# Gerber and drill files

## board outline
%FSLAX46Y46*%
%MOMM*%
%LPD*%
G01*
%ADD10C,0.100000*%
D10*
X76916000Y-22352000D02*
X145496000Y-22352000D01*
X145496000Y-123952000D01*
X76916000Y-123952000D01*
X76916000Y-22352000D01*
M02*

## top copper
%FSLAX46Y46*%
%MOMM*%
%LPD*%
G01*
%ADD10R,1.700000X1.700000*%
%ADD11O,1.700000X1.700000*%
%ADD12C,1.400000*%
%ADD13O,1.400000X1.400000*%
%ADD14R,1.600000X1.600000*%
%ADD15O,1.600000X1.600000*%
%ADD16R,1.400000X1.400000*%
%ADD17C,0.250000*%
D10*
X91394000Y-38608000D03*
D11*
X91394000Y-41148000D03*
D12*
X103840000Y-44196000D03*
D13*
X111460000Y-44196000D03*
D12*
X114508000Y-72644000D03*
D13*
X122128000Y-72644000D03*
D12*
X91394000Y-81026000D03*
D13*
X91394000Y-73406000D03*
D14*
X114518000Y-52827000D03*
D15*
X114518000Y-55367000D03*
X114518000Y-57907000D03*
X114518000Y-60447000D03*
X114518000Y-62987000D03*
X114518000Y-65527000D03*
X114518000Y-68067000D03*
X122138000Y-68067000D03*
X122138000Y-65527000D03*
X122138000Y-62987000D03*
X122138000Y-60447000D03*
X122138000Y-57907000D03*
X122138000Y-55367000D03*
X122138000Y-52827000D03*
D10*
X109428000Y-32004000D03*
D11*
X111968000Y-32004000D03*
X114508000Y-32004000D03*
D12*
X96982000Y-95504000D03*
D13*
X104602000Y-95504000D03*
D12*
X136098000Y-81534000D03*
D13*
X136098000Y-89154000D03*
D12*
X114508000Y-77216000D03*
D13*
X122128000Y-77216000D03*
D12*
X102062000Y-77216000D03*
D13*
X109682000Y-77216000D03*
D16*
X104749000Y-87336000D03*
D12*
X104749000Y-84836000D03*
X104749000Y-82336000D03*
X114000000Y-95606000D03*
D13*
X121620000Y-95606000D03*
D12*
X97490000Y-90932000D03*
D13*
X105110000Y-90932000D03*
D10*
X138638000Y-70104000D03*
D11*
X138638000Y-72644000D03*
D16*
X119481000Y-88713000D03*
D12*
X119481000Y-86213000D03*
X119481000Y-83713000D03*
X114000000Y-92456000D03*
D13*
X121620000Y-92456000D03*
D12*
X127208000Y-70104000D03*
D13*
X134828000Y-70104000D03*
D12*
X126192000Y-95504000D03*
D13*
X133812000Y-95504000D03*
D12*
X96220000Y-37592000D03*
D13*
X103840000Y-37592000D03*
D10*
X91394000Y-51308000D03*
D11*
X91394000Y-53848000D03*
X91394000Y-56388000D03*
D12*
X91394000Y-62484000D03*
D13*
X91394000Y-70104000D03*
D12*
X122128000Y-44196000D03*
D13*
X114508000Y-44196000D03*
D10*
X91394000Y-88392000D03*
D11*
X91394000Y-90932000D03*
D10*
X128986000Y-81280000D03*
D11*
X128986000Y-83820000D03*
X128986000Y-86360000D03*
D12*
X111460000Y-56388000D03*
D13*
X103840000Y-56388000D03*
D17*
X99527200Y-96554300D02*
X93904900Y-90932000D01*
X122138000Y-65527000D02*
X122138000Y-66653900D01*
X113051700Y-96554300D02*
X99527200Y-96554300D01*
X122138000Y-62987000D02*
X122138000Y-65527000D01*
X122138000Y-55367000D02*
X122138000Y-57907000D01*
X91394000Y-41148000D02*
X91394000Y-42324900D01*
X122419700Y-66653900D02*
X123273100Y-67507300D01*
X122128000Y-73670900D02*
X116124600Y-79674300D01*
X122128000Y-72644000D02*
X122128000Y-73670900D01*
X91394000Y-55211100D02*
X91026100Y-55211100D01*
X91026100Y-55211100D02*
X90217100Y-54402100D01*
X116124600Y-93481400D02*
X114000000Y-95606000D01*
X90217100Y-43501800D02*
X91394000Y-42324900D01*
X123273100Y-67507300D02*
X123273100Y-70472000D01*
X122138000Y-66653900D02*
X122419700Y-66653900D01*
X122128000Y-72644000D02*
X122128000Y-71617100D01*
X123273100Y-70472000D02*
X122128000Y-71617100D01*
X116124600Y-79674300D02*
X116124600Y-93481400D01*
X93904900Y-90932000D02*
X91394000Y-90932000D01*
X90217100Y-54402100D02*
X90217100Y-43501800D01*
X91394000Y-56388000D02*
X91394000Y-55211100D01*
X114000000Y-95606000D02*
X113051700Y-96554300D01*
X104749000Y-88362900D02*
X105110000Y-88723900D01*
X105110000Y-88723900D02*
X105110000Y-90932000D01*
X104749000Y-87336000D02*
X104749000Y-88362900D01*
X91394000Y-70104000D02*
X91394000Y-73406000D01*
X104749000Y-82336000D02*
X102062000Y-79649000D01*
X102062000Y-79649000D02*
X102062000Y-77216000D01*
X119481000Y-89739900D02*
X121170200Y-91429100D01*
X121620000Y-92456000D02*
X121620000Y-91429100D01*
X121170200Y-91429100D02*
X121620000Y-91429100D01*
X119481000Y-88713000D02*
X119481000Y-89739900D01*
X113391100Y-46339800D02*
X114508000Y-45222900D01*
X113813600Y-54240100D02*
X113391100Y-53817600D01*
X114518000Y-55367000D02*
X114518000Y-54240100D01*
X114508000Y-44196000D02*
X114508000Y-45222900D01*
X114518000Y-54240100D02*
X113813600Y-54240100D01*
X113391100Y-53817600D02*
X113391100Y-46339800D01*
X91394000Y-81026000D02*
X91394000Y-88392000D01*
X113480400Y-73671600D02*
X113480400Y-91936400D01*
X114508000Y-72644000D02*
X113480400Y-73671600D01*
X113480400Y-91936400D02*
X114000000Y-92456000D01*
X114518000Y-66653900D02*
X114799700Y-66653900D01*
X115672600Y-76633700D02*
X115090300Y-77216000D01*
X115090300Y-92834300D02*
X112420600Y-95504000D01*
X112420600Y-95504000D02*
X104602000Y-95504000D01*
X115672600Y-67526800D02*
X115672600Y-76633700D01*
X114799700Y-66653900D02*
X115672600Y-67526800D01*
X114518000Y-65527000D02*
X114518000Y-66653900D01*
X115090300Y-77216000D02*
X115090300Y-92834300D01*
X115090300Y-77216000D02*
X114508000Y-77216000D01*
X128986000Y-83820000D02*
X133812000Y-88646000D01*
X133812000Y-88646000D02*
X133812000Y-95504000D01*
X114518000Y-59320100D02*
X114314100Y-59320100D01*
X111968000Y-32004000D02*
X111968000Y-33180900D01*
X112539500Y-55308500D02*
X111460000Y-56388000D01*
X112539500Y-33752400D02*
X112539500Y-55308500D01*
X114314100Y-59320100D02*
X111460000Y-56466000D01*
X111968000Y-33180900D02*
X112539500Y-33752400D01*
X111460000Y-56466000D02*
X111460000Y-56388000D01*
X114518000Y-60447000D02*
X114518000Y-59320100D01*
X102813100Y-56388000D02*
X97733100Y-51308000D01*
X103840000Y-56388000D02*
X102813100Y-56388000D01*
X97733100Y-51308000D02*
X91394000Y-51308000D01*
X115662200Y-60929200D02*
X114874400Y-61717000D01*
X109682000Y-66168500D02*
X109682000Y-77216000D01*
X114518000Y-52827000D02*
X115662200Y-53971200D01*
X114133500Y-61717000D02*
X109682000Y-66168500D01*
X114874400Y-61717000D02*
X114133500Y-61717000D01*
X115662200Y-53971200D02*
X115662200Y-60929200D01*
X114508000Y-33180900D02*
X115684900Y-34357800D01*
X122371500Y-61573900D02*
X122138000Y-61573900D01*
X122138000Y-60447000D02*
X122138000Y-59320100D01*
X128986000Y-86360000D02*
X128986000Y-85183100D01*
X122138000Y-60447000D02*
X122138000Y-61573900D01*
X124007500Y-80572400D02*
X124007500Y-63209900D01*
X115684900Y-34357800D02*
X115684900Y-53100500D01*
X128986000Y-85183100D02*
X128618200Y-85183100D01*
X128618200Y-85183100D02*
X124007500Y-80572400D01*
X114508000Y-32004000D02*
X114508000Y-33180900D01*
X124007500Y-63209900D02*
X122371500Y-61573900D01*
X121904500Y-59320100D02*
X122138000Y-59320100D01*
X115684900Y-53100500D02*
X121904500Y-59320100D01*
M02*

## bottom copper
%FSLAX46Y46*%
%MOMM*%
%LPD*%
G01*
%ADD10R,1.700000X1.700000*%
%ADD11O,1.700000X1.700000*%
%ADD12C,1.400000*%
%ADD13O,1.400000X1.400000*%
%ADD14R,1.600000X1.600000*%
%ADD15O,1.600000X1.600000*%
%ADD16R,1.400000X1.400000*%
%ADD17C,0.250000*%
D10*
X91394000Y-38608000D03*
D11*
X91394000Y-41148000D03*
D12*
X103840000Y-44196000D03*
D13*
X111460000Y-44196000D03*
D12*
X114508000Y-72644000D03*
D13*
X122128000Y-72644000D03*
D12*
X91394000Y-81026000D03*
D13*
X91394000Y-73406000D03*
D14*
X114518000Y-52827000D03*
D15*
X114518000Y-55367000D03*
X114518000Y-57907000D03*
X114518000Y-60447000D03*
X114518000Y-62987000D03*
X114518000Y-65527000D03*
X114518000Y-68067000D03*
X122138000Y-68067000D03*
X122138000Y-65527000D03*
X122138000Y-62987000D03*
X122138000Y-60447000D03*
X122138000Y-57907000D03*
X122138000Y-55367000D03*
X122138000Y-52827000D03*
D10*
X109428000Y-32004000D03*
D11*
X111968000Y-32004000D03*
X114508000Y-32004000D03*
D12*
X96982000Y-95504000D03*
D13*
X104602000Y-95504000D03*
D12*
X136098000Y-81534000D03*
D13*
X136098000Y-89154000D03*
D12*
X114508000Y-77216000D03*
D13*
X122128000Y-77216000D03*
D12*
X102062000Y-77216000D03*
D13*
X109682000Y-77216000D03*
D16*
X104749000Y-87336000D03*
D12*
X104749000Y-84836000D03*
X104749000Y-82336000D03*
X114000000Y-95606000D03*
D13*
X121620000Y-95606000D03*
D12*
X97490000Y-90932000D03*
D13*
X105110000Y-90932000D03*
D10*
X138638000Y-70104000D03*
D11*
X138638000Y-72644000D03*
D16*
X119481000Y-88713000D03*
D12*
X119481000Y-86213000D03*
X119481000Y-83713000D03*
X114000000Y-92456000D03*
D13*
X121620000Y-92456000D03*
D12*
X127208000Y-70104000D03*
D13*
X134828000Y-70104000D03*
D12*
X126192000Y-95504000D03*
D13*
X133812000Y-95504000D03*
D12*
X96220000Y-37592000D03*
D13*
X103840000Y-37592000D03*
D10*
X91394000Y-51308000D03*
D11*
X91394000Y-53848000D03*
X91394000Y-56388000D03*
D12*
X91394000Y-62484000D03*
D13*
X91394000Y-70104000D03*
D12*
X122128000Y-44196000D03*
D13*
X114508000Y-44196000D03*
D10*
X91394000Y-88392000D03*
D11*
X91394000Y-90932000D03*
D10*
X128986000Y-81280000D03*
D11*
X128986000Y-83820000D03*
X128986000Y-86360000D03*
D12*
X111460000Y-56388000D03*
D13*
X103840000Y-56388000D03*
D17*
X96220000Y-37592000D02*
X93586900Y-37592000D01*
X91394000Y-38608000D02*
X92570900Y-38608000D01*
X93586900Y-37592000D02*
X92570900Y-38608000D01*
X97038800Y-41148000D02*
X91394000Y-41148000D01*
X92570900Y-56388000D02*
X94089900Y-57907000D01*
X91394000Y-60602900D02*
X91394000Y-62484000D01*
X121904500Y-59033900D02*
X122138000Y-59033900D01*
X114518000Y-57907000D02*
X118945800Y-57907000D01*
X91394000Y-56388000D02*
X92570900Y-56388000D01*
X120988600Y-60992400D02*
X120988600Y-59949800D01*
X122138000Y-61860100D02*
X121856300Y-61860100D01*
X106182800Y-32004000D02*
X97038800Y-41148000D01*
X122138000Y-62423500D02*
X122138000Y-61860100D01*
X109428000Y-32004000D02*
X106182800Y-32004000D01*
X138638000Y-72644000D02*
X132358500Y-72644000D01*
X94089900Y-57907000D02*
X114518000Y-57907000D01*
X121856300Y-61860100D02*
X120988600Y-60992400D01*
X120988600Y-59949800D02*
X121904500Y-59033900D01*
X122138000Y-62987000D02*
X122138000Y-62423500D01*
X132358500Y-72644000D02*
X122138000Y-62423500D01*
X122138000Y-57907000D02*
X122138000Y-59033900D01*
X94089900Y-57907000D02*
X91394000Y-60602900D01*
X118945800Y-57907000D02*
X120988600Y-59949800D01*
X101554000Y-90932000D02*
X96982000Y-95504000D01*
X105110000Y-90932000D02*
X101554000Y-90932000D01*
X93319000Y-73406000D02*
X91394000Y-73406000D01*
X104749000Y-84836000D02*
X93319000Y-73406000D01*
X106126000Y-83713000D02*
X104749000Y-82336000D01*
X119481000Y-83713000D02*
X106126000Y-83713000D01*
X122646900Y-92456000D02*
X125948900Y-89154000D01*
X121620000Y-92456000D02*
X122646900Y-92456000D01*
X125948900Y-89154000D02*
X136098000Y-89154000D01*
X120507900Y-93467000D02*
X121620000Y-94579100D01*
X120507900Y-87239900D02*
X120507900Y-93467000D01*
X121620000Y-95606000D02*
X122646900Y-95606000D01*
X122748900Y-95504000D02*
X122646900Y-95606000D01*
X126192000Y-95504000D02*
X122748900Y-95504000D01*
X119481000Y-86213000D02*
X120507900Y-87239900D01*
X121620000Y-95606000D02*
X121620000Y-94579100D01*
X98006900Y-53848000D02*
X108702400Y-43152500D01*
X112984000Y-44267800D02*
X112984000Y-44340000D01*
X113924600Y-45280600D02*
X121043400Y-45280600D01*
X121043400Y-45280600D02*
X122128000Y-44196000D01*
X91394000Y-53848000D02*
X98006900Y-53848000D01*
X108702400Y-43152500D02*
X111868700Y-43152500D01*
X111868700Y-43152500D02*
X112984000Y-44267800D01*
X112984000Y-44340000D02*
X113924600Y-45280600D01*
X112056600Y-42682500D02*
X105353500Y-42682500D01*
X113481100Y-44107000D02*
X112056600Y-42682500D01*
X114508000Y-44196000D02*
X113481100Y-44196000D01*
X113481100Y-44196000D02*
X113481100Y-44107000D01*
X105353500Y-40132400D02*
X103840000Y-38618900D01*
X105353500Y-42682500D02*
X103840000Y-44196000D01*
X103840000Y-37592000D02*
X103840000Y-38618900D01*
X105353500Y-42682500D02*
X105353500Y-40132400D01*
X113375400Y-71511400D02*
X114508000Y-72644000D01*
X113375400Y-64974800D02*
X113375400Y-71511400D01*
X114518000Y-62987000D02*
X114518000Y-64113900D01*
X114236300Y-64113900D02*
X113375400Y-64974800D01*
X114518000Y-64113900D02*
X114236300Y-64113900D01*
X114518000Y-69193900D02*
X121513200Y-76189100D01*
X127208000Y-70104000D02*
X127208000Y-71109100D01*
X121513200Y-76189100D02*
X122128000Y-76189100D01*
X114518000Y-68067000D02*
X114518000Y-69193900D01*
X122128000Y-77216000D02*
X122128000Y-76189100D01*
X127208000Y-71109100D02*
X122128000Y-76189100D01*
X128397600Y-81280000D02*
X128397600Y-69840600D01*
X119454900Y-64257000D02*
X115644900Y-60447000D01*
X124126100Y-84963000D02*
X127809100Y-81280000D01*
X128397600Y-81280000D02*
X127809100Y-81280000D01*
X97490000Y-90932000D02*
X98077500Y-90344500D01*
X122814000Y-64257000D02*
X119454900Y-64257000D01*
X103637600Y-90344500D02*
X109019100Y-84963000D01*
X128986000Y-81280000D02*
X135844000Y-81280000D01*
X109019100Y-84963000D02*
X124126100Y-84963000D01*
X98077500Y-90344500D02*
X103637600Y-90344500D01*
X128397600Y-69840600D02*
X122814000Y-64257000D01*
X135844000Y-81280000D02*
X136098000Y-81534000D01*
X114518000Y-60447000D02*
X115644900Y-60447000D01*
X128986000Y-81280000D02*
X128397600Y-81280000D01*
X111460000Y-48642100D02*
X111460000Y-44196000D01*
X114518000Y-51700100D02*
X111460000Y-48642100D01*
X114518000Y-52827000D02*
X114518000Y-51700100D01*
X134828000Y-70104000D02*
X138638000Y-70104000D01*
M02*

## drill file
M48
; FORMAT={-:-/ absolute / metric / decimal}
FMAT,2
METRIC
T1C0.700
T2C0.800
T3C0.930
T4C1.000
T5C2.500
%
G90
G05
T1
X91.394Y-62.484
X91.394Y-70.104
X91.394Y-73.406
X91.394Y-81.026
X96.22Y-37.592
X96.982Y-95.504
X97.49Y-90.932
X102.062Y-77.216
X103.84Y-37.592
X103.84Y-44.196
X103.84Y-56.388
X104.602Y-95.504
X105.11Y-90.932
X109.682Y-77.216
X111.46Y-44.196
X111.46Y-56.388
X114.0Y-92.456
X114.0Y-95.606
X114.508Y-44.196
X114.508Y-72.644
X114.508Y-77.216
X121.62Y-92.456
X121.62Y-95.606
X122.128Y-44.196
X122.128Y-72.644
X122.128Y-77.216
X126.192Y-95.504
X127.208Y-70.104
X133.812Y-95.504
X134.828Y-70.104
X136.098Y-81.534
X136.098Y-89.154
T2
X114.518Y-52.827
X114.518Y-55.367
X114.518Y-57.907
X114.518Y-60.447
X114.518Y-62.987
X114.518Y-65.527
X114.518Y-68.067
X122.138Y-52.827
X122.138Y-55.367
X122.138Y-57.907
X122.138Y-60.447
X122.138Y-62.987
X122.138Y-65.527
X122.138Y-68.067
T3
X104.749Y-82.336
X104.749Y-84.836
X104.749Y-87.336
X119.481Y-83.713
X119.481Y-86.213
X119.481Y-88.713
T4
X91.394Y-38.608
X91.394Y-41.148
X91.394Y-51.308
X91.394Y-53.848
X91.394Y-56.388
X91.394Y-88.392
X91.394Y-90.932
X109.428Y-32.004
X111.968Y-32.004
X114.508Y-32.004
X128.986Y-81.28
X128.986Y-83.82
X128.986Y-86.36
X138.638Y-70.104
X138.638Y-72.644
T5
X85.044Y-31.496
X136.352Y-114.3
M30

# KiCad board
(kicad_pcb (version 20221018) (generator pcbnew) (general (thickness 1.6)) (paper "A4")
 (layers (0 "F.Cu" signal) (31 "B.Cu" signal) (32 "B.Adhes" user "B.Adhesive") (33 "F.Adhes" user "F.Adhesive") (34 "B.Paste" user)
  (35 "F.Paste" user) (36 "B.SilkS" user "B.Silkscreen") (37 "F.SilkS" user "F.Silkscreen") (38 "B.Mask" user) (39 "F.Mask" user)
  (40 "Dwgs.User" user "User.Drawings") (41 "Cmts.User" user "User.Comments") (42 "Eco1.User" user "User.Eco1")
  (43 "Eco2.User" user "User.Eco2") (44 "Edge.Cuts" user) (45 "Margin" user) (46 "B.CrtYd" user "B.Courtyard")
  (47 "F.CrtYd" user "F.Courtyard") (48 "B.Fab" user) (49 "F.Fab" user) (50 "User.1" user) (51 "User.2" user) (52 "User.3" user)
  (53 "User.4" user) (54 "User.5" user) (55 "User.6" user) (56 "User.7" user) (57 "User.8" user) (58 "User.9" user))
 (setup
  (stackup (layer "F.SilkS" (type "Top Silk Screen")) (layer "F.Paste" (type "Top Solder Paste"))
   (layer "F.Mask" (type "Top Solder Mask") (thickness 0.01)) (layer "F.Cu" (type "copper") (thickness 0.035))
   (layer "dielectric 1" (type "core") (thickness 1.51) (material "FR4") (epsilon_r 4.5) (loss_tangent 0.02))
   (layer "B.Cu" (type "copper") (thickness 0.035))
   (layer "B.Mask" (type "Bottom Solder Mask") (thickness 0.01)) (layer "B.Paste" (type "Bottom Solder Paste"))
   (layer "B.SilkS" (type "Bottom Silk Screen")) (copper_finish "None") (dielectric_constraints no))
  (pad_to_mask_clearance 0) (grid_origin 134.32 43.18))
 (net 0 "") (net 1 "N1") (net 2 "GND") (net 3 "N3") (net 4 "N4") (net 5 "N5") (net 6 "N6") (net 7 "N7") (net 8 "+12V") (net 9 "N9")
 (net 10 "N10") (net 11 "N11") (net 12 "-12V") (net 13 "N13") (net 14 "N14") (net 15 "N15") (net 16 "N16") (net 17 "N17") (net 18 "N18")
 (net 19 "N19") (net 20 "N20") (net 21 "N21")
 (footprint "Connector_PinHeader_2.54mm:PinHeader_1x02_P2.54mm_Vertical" (layer "F.Cu") (at 91.394 38.608)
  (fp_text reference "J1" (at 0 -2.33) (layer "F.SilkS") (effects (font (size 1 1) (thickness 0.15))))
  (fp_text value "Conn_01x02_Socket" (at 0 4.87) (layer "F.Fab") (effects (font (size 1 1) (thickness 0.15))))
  (pad "1" thru_hole rect (at 0 0) (size 1.7 1.7) (drill 1) (layers "*.Cu" "*.Mask") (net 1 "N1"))
  (pad "2" thru_hole oval (at 0 2.54) (size 1.7 1.7) (drill 1) (layers "*.Cu" "*.Mask") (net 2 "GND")))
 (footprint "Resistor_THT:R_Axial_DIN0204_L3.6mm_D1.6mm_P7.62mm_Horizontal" (layer "F.Cu") (at 103.84 44.196)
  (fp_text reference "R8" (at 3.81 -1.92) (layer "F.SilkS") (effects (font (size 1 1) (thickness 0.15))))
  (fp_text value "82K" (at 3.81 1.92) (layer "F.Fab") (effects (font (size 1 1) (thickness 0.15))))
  (pad "1" thru_hole circle (at 0 0) (size 1.4 1.4) (drill 0.7) (layers "*.Cu" "*.Mask") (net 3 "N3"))
  (pad "2" thru_hole oval (at 7.62 0) (size 1.4 1.4) (drill 0.7) (layers "*.Cu" "*.Mask") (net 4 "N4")))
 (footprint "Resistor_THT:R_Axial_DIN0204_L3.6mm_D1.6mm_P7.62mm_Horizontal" (layer "F.Cu") (at 114.508 72.644)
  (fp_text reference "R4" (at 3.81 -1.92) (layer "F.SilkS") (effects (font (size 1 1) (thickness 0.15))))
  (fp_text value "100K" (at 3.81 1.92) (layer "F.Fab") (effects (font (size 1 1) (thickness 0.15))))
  (pad "1" thru_hole circle (at 0 0) (size 1.4 1.4) (drill 0.7) (layers "*.Cu" "*.Mask") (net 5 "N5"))
  (pad "2" thru_hole oval (at 7.62 0) (size 1.4 1.4) (drill 0.7) (layers "*.Cu" "*.Mask") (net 2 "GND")))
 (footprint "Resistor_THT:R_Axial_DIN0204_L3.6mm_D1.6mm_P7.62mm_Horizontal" (layer "F.Cu") (at 91.394 81.026 90)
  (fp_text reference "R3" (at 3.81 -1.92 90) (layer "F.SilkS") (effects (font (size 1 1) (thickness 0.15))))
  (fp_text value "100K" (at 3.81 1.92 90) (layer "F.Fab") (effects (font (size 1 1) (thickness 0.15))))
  (pad "1" thru_hole circle (at 0 0 90) (size 1.4 1.4) (drill 0.7) (layers "*.Cu" "*.Mask") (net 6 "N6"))
  (pad "2" thru_hole oval (at 7.62 0 90) (size 1.4 1.4) (drill 0.7) (layers "*.Cu" "*.Mask") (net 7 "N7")))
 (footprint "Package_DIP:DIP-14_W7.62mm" (layer "F.Cu") (at 114.518 52.827)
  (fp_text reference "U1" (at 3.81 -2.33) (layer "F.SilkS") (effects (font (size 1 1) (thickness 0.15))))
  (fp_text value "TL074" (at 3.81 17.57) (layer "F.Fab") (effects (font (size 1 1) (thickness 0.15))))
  (pad "1" thru_hole rect (at 0 0) (size 1.6 1.6) (drill 0.8) (layers "*.Cu" "*.Mask") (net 4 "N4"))
  (pad "2" thru_hole oval (at 0 2.54) (size 1.6 1.6) (drill 0.8) (layers "*.Cu" "*.Mask") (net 3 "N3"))
  (pad "3" thru_hole oval (at 0 5.08) (size 1.6 1.6) (drill 0.8) (layers "*.Cu" "*.Mask") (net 2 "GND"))
  (pad "4" thru_hole oval (at 0 7.62) (size 1.6 1.6) (drill 0.8) (layers "*.Cu" "*.Mask") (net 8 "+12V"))
  (pad "5" thru_hole oval (at 0 10.16) (size 1.6 1.6) (drill 0.8) (layers "*.Cu" "*.Mask") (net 5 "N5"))
  (pad "6" thru_hole oval (at 0 12.7) (size 1.6 1.6) (drill 0.8) (layers "*.Cu" "*.Mask") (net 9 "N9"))
  (pad "7" thru_hole oval (at 0 15.24) (size 1.6 1.6) (drill 0.8) (layers "*.Cu" "*.Mask") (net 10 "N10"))
  (pad "8" thru_hole oval (at 7.62 15.24) (size 1.6 1.6) (drill 0.8) (layers "*.Cu" "*.Mask") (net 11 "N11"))
  (pad "9" thru_hole oval (at 7.62 12.7) (size 1.6 1.6) (drill 0.8) (layers "*.Cu" "*.Mask") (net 2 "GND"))
  (pad "10" thru_hole oval (at 7.62 10.16) (size 1.6 1.6) (drill 0.8) (layers "*.Cu" "*.Mask") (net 2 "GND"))
  (pad "11" thru_hole oval (at 7.62 7.62) (size 1.6 1.6) (drill 0.8) (layers "*.Cu" "*.Mask") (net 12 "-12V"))
  (pad "12" thru_hole oval (at 7.62 5.08) (size 1.6 1.6) (drill 0.8) (layers "*.Cu" "*.Mask") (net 2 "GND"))
  (pad "13" thru_hole oval (at 7.62 2.54) (size 1.6 1.6) (drill 0.8) (layers "*.Cu" "*.Mask") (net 2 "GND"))
  (pad "14" thru_hole oval (at 7.62 0) (size 1.6 1.6) (drill 0.8) (layers "*.Cu" "*.Mask") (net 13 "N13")))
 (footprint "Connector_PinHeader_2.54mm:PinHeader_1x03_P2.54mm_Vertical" (layer "F.Cu") (at 109.428 32.004 90)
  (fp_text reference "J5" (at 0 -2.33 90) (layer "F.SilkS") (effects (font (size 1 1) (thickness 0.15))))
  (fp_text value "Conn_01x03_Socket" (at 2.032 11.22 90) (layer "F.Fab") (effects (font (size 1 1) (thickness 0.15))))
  (pad "1" thru_hole rect (at 0 0 90) (size 1.7 1.7) (drill 1) (layers "*.Cu" "*.Mask") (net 2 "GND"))
  (pad "2" thru_hole oval (at 0 2.54 90) (size 1.7 1.7) (drill 1) (layers "*.Cu" "*.Mask") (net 8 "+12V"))
  (pad "3" thru_hole oval (at 0 5.08 90) (size 1.7 1.7) (drill 1) (layers "*.Cu" "*.Mask") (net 12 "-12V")))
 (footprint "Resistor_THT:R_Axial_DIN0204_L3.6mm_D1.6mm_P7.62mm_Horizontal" (layer "F.Cu") (at 96.982 95.504)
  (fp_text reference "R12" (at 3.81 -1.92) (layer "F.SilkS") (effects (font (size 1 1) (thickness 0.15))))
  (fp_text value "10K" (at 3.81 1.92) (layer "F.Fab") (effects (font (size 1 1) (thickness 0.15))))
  (pad "1" thru_hole circle (at 0 0) (size 1.4 1.4) (drill 0.7) (layers "*.Cu" "*.Mask") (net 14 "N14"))
  (pad "2" thru_hole oval (at 7.62 0) (size 1.4 1.4) (drill 0.7) (layers "*.Cu" "*.Mask") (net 9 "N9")))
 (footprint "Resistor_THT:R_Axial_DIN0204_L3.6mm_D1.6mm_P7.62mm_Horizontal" (layer "F.Cu") (at 136.098 81.534 -90)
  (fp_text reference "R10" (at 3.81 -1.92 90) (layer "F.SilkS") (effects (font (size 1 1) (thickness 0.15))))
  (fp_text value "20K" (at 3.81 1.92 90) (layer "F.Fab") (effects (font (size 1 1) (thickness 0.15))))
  (pad "1" thru_hole circle (at 0 0 270) (size 1.4 1.4) (drill 0.7) (layers "*.Cu" "*.Mask") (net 8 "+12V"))
  (pad "2" thru_hole oval (at 7.62 0 270) (size 1.4 1.4) (drill 0.7) (layers "*.Cu" "*.Mask") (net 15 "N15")))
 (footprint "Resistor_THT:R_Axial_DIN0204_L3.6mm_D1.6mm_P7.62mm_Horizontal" (layer "F.Cu") (at 114.508 77.216)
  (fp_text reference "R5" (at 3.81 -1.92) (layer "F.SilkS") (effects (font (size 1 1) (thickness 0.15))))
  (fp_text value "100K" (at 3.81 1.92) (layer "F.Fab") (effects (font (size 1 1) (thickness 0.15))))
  (pad "1" thru_hole circle (at 0 0) (size 1.4 1.4) (drill 0.7) (layers "*.Cu" "*.Mask") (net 9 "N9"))
  (pad "2" thru_hole oval (at 7.62 0) (size 1.4 1.4) (drill 0.7) (layers "*.Cu" "*.Mask") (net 10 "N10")))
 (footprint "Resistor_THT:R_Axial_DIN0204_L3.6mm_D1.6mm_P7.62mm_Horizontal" (layer "F.Cu") (at 102.062 77.216)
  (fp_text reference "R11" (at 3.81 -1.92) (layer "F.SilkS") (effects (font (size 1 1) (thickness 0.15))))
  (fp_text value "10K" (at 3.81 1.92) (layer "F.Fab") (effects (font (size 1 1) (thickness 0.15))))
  (pad "1" thru_hole circle (at 0 0) (size 1.4 1.4) (drill 0.7) (layers "*.Cu" "*.Mask") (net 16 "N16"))
  (pad "2" thru_hole oval (at 7.62 0) (size 1.4 1.4) (drill 0.7) (layers "*.Cu" "*.Mask") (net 4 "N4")))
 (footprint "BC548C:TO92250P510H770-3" (layer "F.Cu") (at 104.094 84.836 90)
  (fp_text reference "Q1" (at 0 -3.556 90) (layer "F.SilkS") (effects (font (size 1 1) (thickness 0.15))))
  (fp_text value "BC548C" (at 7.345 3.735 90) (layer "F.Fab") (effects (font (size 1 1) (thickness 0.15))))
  (pad "1" thru_hole rect (at -2.5 0.655 90) (size 1.4 1.4) (drill 0.93) (layers "*.Cu" "*.Mask") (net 14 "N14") (solder_mask_margin 0.102))
  (pad "2" thru_hole circle (at 0 0.655 90) (size 1.4 1.4) (drill 0.93) (layers "*.Cu" "*.Mask") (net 7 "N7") (solder_mask_margin 0.102))
  (pad "3" thru_hole circle (at 2.5 0.655 90) (size 1.4 1.4) (drill 0.93) (layers "*.Cu" "*.Mask") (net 16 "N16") (solder_mask_margin 0.102)))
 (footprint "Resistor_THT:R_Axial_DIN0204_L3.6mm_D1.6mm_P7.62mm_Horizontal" (layer "F.Cu") (at 114 95.606)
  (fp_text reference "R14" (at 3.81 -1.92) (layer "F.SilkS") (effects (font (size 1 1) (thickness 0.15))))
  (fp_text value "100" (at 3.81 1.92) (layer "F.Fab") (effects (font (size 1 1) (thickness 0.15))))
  (pad "1" thru_hole circle (at 0 0) (size 1.4 1.4) (drill 0.7) (layers "*.Cu" "*.Mask") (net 2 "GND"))
  (pad "2" thru_hole oval (at 7.62 0) (size 1.4 1.4) (drill 0.7) (layers "*.Cu" "*.Mask") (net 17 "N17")))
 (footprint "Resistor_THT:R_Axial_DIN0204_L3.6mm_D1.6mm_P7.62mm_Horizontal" (layer "F.Cu") (at 97.49 90.932)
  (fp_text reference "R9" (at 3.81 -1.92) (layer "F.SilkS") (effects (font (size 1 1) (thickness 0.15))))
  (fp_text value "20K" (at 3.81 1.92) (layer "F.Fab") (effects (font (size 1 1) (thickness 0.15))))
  (pad "1" thru_hole circle (at 0 0) (size 1.4 1.4) (drill 0.7) (layers "*.Cu" "*.Mask") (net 8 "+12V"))
  (pad "2" thru_hole oval (at 7.62 0) (size 1.4 1.4) (drill 0.7) (layers "*.Cu" "*.Mask") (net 14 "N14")))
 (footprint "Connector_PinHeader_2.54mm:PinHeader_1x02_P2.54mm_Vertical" (layer "F.Cu") (at 138.638 70.104)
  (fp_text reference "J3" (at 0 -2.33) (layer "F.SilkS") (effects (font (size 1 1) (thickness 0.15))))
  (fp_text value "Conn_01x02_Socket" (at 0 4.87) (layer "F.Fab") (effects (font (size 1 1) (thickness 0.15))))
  (pad "1" thru_hole rect (at 0 0) (size 1.7 1.7) (drill 1) (layers "*.Cu" "*.Mask") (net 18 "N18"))
  (pad "2" thru_hole oval (at 0 2.54) (size 1.7 1.7) (drill 1) (layers "*.Cu" "*.Mask") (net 2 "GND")))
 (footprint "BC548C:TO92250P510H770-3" (layer "F.Cu") (at 118.826 86.213 90)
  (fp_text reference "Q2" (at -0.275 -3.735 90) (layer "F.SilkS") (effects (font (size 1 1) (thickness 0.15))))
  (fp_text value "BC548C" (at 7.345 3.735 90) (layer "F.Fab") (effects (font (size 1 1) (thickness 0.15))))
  (pad "1" thru_hole rect (at -2.5 0.655 90) (size 1.4 1.4) (drill 0.93) (layers "*.Cu" "*.Mask") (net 15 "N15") (solder_mask_margin 0.102))
  (pad "2" thru_hole circle (at 0 0.655 90) (size 1.4 1.4) (drill 0.93) (layers "*.Cu" "*.Mask") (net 17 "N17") (solder_mask_margin 0.102))
  (pad "3" thru_hole circle (at 2.5 0.655 90) (size 1.4 1.4) (drill 0.93) (layers "*.Cu" "*.Mask") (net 16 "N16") (solder_mask_margin 0.102)))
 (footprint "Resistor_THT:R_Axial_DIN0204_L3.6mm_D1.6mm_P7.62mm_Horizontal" (layer "F.Cu") (at 114 92.456)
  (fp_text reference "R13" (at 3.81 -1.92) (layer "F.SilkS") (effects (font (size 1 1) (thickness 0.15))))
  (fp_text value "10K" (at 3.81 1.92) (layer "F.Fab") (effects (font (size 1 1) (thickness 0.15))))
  (pad "1" thru_hole circle (at 0 0) (size 1.4 1.4) (drill 0.7) (layers "*.Cu" "*.Mask") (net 5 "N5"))
  (pad "2" thru_hole oval (at 7.62 0) (size 1.4 1.4) (drill 0.7) (layers "*.Cu" "*.Mask") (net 15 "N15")))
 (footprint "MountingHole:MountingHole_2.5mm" (layer "F.Cu") (at 85.044 31.496)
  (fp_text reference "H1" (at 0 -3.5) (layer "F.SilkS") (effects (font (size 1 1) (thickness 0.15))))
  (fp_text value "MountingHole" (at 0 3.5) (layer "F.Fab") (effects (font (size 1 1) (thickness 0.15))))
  (pad "" np_thru_hole circle (at 0 0) (size 2.5 2.5) (drill 2.5) (layers "*.Cu" "*.Mask")))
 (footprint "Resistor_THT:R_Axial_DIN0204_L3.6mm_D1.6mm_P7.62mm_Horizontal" (layer "F.Cu") (at 127.208 70.104)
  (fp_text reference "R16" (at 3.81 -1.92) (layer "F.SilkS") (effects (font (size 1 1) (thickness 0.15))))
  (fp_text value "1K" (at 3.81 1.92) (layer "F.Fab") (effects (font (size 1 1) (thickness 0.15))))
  (pad "1" thru_hole circle (at 0 0) (size 1.4 1.4) (drill 0.7) (layers "*.Cu" "*.Mask") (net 10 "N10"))
  (pad "2" thru_hole oval (at 7.62 0) (size 1.4 1.4) (drill 0.7) (layers "*.Cu" "*.Mask") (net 18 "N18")))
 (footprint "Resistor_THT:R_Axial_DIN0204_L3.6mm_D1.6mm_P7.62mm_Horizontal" (layer "F.Cu") (at 126.192 95.504)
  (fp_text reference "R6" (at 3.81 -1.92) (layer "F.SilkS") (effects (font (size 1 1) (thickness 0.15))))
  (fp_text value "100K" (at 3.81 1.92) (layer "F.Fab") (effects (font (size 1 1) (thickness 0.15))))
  (pad "1" thru_hole circle (at 0 0) (size 1.4 1.4) (drill 0.7) (layers "*.Cu" "*.Mask") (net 17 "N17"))
  (pad "2" thru_hole oval (at 7.62 0) (size 1.4 1.4) (drill 0.7) (layers "*.Cu" "*.Mask") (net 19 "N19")))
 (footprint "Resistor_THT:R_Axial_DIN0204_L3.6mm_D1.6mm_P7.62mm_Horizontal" (layer "F.Cu") (at 96.22 37.592)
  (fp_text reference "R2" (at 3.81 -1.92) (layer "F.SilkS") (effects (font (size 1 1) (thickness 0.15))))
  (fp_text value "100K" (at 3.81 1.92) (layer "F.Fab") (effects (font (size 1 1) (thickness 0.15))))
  (pad "1" thru_hole circle (at 0 0) (size 1.4 1.4) (drill 0.7) (layers "*.Cu" "*.Mask") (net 1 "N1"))
  (pad "2" thru_hole oval (at 7.62 0) (size 1.4 1.4) (drill 0.7) (layers "*.Cu" "*.Mask") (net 3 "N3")))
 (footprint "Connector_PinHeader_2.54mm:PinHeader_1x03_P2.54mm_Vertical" (layer "F.Cu") (at 91.394 51.308)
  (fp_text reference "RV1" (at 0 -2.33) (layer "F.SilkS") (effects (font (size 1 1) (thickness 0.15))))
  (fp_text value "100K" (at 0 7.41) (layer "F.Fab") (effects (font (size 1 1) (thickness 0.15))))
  (pad "1" thru_hole rect (at 0 0) (size 1.7 1.7) (drill 1) (layers "*.Cu" "*.Mask") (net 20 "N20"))
  (pad "2" thru_hole oval (at 0 2.54) (size 1.7 1.7) (drill 1) (layers "*.Cu" "*.Mask") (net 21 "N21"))
  (pad "3" thru_hole oval (at 0 5.08) (size 1.7 1.7) (drill 1) (layers "*.Cu" "*.Mask") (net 2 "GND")))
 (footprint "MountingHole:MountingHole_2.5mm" (layer "F.Cu") (at 136.352 114.3)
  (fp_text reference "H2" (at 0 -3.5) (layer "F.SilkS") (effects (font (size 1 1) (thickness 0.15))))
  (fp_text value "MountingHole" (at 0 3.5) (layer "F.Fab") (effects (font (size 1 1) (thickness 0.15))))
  (pad "" np_thru_hole circle (at 0 0) (size 2.5 2.5) (drill 2.5) (layers "*.Cu" "*.Mask")))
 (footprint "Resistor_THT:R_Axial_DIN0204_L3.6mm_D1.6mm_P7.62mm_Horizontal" (layer "F.Cu") (at 91.394 62.484 -90)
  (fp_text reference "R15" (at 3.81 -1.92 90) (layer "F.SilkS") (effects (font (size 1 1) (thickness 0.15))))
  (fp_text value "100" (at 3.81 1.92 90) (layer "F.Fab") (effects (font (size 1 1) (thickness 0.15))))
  (pad "1" thru_hole circle (at 0 0 270) (size 1.4 1.4) (drill 0.7) (layers "*.Cu" "*.Mask") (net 2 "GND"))
  (pad "2" thru_hole oval (at 7.62 0 270) (size 1.4 1.4) (drill 0.7) (layers "*.Cu" "*.Mask") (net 7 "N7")))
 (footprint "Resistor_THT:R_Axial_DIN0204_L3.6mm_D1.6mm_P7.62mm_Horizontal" (layer "F.Cu") (at 122.128 44.196 180)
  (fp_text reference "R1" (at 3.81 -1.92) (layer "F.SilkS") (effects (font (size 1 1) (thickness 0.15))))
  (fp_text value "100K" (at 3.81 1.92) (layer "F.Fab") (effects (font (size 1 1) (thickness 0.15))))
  (pad "1" thru_hole circle (at 0 0 180) (size 1.4 1.4) (drill 0.7) (layers "*.Cu" "*.Mask") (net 21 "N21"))
  (pad "2" thru_hole oval (at 7.62 0 180) (size 1.4 1.4) (drill 0.7) (layers "*.Cu" "*.Mask") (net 3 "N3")))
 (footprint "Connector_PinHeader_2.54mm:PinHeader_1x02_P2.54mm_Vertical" (layer "F.Cu") (at 91.394 88.392)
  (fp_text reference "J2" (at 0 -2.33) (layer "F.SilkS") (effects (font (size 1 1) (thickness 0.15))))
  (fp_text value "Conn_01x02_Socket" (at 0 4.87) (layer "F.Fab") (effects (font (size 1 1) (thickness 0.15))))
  (pad "1" thru_hole rect (at 0 0) (size 1.7 1.7) (drill 1) (layers "*.Cu" "*.Mask") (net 6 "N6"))
  (pad "2" thru_hole oval (at 0 2.54) (size 1.7 1.7) (drill 1) (layers "*.Cu" "*.Mask") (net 2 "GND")))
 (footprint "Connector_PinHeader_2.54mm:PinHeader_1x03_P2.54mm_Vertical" (layer "F.Cu") (at 128.986 81.28)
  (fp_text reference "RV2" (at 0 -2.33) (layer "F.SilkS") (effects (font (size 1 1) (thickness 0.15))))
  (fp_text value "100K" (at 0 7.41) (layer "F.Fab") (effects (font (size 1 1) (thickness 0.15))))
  (pad "1" thru_hole rect (at 0 0) (size 1.7 1.7) (drill 1) (layers "*.Cu" "*.Mask") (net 8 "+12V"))
  (pad "2" thru_hole oval (at 0 2.54) (size 1.7 1.7) (drill 1) (layers "*.Cu" "*.Mask") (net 19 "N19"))
  (pad "3" thru_hole oval (at 0 5.08) (size 1.7 1.7) (drill 1) (layers "*.Cu" "*.Mask") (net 12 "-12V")))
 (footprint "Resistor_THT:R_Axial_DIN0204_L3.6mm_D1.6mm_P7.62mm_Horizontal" (layer "F.Cu") (at 111.46 56.388 180)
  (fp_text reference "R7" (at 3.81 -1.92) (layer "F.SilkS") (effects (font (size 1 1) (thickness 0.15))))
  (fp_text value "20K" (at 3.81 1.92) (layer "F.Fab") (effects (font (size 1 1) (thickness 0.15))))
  (pad "1" thru_hole circle (at 0 0 180) (size 1.4 1.4) (drill 0.7) (layers "*.Cu" "*.Mask") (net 8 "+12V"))
  (pad "2" thru_hole oval (at 7.62 0 180) (size 1.4 1.4) (drill 0.7) (layers "*.Cu" "*.Mask") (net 20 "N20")))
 (gr_rect (start 76.916 22.352) (end 145.496 123.952) (stroke (width 0.1) (type default)) (fill none) (layer "Edge.Cuts"))
 (segment (start 96.22 37.592) (end 93.5869 37.592) (width 0.25) (layer "B.Cu") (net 1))
 (segment (start 91.394 38.608) (end 92.5709 38.608) (width 0.25) (layer "B.Cu") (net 1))
 (segment (start 93.5869 37.592) (end 92.5709 38.608) (width 0.25) (layer "B.Cu") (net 1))
 (segment (start 99.5272 96.5543) (end 93.9049 90.932) (width 0.25) (layer "F.Cu") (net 2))
 (segment (start 122.138 65.527) (end 122.138 66.6539) (width 0.25) (layer "F.Cu") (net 2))
 (segment (start 113.0517 96.5543) (end 99.5272 96.5543) (width 0.25) (layer "F.Cu") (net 2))
 (segment (start 122.138 62.987) (end 122.138 65.527) (width 0.25) (layer "F.Cu") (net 2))
 (segment (start 122.138 55.367) (end 122.138 57.907) (width 0.25) (layer "F.Cu") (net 2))
 (segment (start 91.394 41.148) (end 91.394 42.3249) (width 0.25) (layer "F.Cu") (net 2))
 (segment (start 122.4197 66.6539) (end 123.2731 67.5073) (width 0.25) (layer "F.Cu") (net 2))
 (segment (start 122.128 73.6709) (end 116.1246 79.6743) (width 0.25) (layer "F.Cu") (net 2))
 (segment (start 122.128 72.644) (end 122.128 73.6709) (width 0.25) (layer "F.Cu") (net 2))
 (segment (start 91.394 55.2111) (end 91.0261 55.2111) (width 0.25) (layer "F.Cu") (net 2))
 (segment (start 91.0261 55.2111) (end 90.2171 54.4021) (width 0.25) (layer "F.Cu") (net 2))
 (segment (start 116.1246 93.4814) (end 114 95.606) (width 0.25) (layer "F.Cu") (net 2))
 (segment (start 90.2171 43.5018) (end 91.394 42.3249) (width 0.25) (layer "F.Cu") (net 2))
 (segment (start 123.2731 67.5073) (end 123.2731 70.472) (width 0.25) (layer "F.Cu") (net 2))
 (segment (start 122.138 66.6539) (end 122.4197 66.6539) (width 0.25) (layer "F.Cu") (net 2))
 (segment (start 122.128 72.644) (end 122.128 71.6171) (width 0.25) (layer "F.Cu") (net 2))
 (segment (start 123.2731 70.472) (end 122.128 71.6171) (width 0.25) (layer "F.Cu") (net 2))
 (segment (start 116.1246 79.6743) (end 116.1246 93.4814) (width 0.25) (layer "F.Cu") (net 2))
 (segment (start 93.9049 90.932) (end 91.394 90.932) (width 0.25) (layer "F.Cu") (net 2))
 (segment (start 90.2171 54.4021) (end 90.2171 43.5018) (width 0.25) (layer "F.Cu") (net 2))
 (segment (start 91.394 56.388) (end 91.394 55.2111) (width 0.25) (layer "F.Cu") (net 2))
 (segment (start 114 95.606) (end 113.0517 96.5543) (width 0.25) (layer "F.Cu") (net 2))
 (segment (start 97.0388 41.148) (end 91.394 41.148) (width 0.25) (layer "B.Cu") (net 2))
 (segment (start 92.5709 56.388) (end 94.0899 57.907) (width 0.25) (layer "B.Cu") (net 2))
 (segment (start 91.394 60.6029) (end 91.394 62.484) (width 0.25) (layer "B.Cu") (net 2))
 (segment (start 121.9045 59.0339) (end 122.138 59.0339) (width 0.25) (layer "B.Cu") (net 2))
 (segment (start 114.518 57.907) (end 118.9458 57.907) (width 0.25) (layer "B.Cu") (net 2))
 (segment (start 91.394 56.388) (end 92.5709 56.388) (width 0.25) (layer "B.Cu") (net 2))
 (segment (start 120.9886 60.9924) (end 120.9886 59.9498) (width 0.25) (layer "B.Cu") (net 2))
 (segment (start 122.138 61.8601) (end 121.8563 61.8601) (width 0.25) (layer "B.Cu") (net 2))
 (segment (start 106.1828 32.004) (end 97.0388 41.148) (width 0.25) (layer "B.Cu") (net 2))
 (segment (start 122.138 62.4235) (end 122.138 61.8601) (width 0.25) (layer "B.Cu") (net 2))
 (segment (start 109.428 32.004) (end 106.1828 32.004) (width 0.25) (layer "B.Cu") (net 2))
 (segment (start 138.638 72.644) (end 132.3585 72.644) (width 0.25) (layer "B.Cu") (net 2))
 (segment (start 94.0899 57.907) (end 114.518 57.907) (width 0.25) (layer "B.Cu") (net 2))
 (segment (start 121.8563 61.8601) (end 120.9886 60.9924) (width 0.25) (layer "B.Cu") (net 2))
 (segment (start 120.9886 59.9498) (end 121.9045 59.0339) (width 0.25) (layer "B.Cu") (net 2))
 (segment (start 122.138 62.987) (end 122.138 62.4235) (width 0.25) (layer "B.Cu") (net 2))
 (segment (start 132.3585 72.644) (end 122.138 62.4235) (width 0.25) (layer "B.Cu") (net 2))
 (segment (start 122.138 57.907) (end 122.138 59.0339) (width 0.25) (layer "B.Cu") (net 2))
 (segment (start 94.0899 57.907) (end 91.394 60.6029) (width 0.25) (layer "B.Cu") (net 2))
 (segment (start 118.9458 57.907) (end 120.9886 59.9498) (width 0.25) (layer "B.Cu") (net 2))
 (segment (start 104.749 88.3629) (end 105.11 88.7239) (width 0.25) (layer "F.Cu") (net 14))
 (segment (start 105.11 88.7239) (end 105.11 90.932) (width 0.25) (layer "F.Cu") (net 14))
 (segment (start 104.749 87.336) (end 104.749 88.3629) (width 0.25) (layer "F.Cu") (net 14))
 (segment (start 101.554 90.932) (end 96.982 95.504) (width 0.25) (layer "B.Cu") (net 14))
 (segment (start 105.11 90.932) (end 101.554 90.932) (width 0.25) (layer "B.Cu") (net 14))
 (segment (start 91.394 70.104) (end 91.394 73.406) (width 0.25) (layer "F.Cu") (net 7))
 (segment (start 93.319 73.406) (end 91.394 73.406) (width 0.25) (layer "B.Cu") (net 7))
 (segment (start 104.749 84.836) (end 93.319 73.406) (width 0.25) (layer "B.Cu") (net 7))
 (segment (start 104.749 82.336) (end 102.062 79.649) (width 0.25) (layer "F.Cu") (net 16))
 (segment (start 102.062 79.649) (end 102.062 77.216) (width 0.25) (layer "F.Cu") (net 16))
 (segment (start 106.126 83.713) (end 104.749 82.336) (width 0.25) (layer "B.Cu") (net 16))
 (segment (start 119.481 83.713) (end 106.126 83.713) (width 0.25) (layer "B.Cu") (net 16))
 (segment (start 119.481 89.7399) (end 121.1702 91.4291) (width 0.25) (layer "F.Cu") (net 15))
 (segment (start 121.62 92.456) (end 121.62 91.4291) (width 0.25) (layer "F.Cu") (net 15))
 (segment (start 121.1702 91.4291) (end 121.62 91.4291) (width 0.25) (layer "F.Cu") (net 15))
 (segment (start 119.481 88.713) (end 119.481 89.7399) (width 0.25) (layer "F.Cu") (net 15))
 (segment (start 122.6469 92.456) (end 125.9489 89.154) (width 0.25) (layer "B.Cu") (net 15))
 (segment (start 121.62 92.456) (end 122.6469 92.456) (width 0.25) (layer "B.Cu") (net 15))
 (segment (start 125.9489 89.154) (end 136.098 89.154) (width 0.25) (layer "B.Cu") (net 15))
 (segment (start 120.5079 93.467) (end 121.62 94.5791) (width 0.25) (layer "B.Cu") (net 17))
 (segment (start 120.5079 87.2399) (end 120.5079 93.467) (width 0.25) (layer "B.Cu") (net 17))
 (segment (start 121.62 95.606) (end 122.6469 95.606) (width 0.25) (layer "B.Cu") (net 17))
 (segment (start 122.7489 95.504) (end 122.6469 95.606) (width 0.25) (layer "B.Cu") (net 17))
 (segment (start 126.192 95.504) (end 122.7489 95.504) (width 0.25) (layer "B.Cu") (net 17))
 (segment (start 119.481 86.213) (end 120.5079 87.2399) (width 0.25) (layer "B.Cu") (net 17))
 (segment (start 121.62 95.606) (end 121.62 94.5791) (width 0.25) (layer "B.Cu") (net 17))
 (segment (start 98.0069 53.848) (end 108.7024 43.1525) (width 0.25) (layer "B.Cu") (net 21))
 (segment (start 112.984 44.2678) (end 112.984 44.34) (width 0.25) (layer "B.Cu") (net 21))
 (segment (start 113.9246 45.2806) (end 121.0434 45.2806) (width 0.25) (layer "B.Cu") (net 21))
 (segment (start 121.0434 45.2806) (end 122.128 44.196) (width 0.25) (layer "B.Cu") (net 21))
 (segment (start 91.394 53.848) (end 98.0069 53.848) (width 0.25) (layer "B.Cu") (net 21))
 (segment (start 108.7024 43.1525) (end 111.8687 43.1525) (width 0.25) (layer "B.Cu") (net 21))
 (segment (start 111.8687 43.1525) (end 112.984 44.2678) (width 0.25) (layer "B.Cu") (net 21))
 (segment (start 112.984 44.34) (end 113.9246 45.2806) (width 0.25) (layer "B.Cu") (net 21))
 (segment (start 113.3911 46.3398) (end 114.508 45.2229) (width 0.25) (layer "F.Cu") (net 3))
 (segment (start 113.8136 54.2401) (end 113.3911 53.8176) (width 0.25) (layer "F.Cu") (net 3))
 (segment (start 114.518 55.367) (end 114.518 54.2401) (width 0.25) (layer "F.Cu") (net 3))
 (segment (start 114.508 44.196) (end 114.508 45.2229) (width 0.25) (layer "F.Cu") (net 3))
 (segment (start 114.518 54.2401) (end 113.8136 54.2401) (width 0.25) (layer "F.Cu") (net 3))
 (segment (start 113.3911 53.8176) (end 113.3911 46.3398) (width 0.25) (layer "F.Cu") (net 3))
 (segment (start 112.0566 42.6825) (end 105.3535 42.6825) (width 0.25) (layer "B.Cu") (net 3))
 (segment (start 113.4811 44.107) (end 112.0566 42.6825) (width 0.25) (layer "B.Cu") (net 3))
 (segment (start 114.508 44.196) (end 113.4811 44.196) (width 0.25) (layer "B.Cu") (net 3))
 (segment (start 113.4811 44.196) (end 113.4811 44.107) (width 0.25) (layer "B.Cu") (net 3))
 (segment (start 105.3535 40.1324) (end 103.84 38.6189) (width 0.25) (layer "B.Cu") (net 3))
 (segment (start 105.3535 42.6825) (end 103.84 44.196) (width 0.25) (layer "B.Cu") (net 3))
 (segment (start 103.84 37.592) (end 103.84 38.6189) (width 0.25) (layer "B.Cu") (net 3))
 (segment (start 105.3535 42.6825) (end 105.3535 40.1324) (width 0.25) (layer "B.Cu") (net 3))
 (segment (start 91.394 81.026) (end 91.394 88.392) (width 0.25) (layer "F.Cu") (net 6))
 (segment (start 113.4804 73.6716) (end 113.4804 91.9364) (width 0.25) (layer "F.Cu") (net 5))
 (segment (start 114.508 72.644) (end 113.4804 73.6716) (width 0.25) (layer "F.Cu") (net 5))
 (segment (start 113.4804 91.9364) (end 114 92.456) (width 0.25) (layer "F.Cu") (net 5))
 (segment (start 113.3754 71.5114) (end 114.508 72.644) (width 0.25) (layer "B.Cu") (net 5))
 (segment (start 113.3754 64.9748) (end 113.3754 71.5114) (width 0.25) (layer "B.Cu") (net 5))
 (segment (start 114.518 62.987) (end 114.518 64.1139) (width 0.25) (layer "B.Cu") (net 5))
 (segment (start 114.2363 64.1139) (end 113.3754 64.9748) (width 0.25) (layer "B.Cu") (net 5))
 (segment (start 114.518 64.1139) (end 114.2363 64.1139) (width 0.25) (layer "B.Cu") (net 5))
 (segment (start 114.518 66.6539) (end 114.7997 66.6539) (width 0.25) (layer "F.Cu") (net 9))
 (segment (start 115.6726 76.6337) (end 115.0903 77.216) (width 0.25) (layer "F.Cu") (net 9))
 (segment (start 115.0903 92.8343) (end 112.4206 95.504) (width 0.25) (layer "F.Cu") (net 9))
 (segment (start 112.4206 95.504) (end 104.602 95.504) (width 0.25) (layer "F.Cu") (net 9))
 (segment (start 115.6726 67.5268) (end 115.6726 76.6337) (width 0.25) (layer "F.Cu") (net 9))
 (segment (start 114.7997 66.6539) (end 115.6726 67.5268) (width 0.25) (layer "F.Cu") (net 9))
 (segment (start 114.518 65.527) (end 114.518 66.6539) (width 0.25) (layer "F.Cu") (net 9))
 (segment (start 115.0903 77.216) (end 115.0903 92.8343) (width 0.25) (layer "F.Cu") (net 9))
 (segment (start 115.0903 77.216) (end 114.508 77.216) (width 0.25) (layer "F.Cu") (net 9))
 (segment (start 114.518 69.1939) (end 121.5132 76.1891) (width 0.25) (layer "B.Cu") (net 10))
 (segment (start 127.208 70.104) (end 127.208 71.1091) (width 0.25) (layer "B.Cu") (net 10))
 (segment (start 121.5132 76.1891) (end 122.128 76.1891) (width 0.25) (layer "B.Cu") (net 10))
 (segment (start 114.518 68.067) (end 114.518 69.1939) (width 0.25) (layer "B.Cu") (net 10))
 (segment (start 122.128 77.216) (end 122.128 76.1891) (width 0.25) (layer "B.Cu") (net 10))
 (segment (start 127.208 71.1091) (end 122.128 76.1891) (width 0.25) (layer "B.Cu") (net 10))
 (segment (start 128.986 83.82) (end 133.812 88.646) (width 0.25) (layer "F.Cu") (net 19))
 (segment (start 133.812 88.646) (end 133.812 95.504) (width 0.25) (layer "F.Cu") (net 19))
 (segment (start 114.518 59.3201) (end 114.3141 59.3201) (width 0.25) (layer "F.Cu") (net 8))
 (segment (start 111.968 32.004) (end 111.968 33.1809) (width 0.25) (layer "F.Cu") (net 8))
 (segment (start 112.5395 55.3085) (end 111.46 56.388) (width 0.25) (layer "F.Cu") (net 8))
 (segment (start 112.5395 33.7524) (end 112.5395 55.3085) (width 0.25) (layer "F.Cu") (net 8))
 (segment (start 114.3141 59.3201) (end 111.46 56.466) (width 0.25) (layer "F.Cu") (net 8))
 (segment (start 111.968 33.1809) (end 112.5395 33.7524) (width 0.25) (layer "F.Cu") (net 8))
 (segment (start 111.46 56.466) (end 111.46 56.388) (width 0.25) (layer "F.Cu") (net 8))
 (segment (start 114.518 60.447) (end 114.518 59.3201) (width 0.25) (layer "F.Cu") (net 8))
 (segment (start 128.3976 81.28) (end 128.3976 69.8406) (width 0.25) (layer "B.Cu") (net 8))
 (segment (start 119.4549 64.257) (end 115.6449 60.447) (width 0.25) (layer "B.Cu") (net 8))
 (segment (start 124.1261 84.963) (end 127.8091 81.28) (width 0.25) (layer "B.Cu") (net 8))
 (segment (start 128.3976 81.28) (end 127.8091 81.28) (width 0.25) (layer "B.Cu") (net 8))
 (segment (start 97.49 90.932) (end 98.0775 90.3445) (width 0.25) (layer "B.Cu") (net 8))
 (segment (start 122.814 64.257) (end 119.4549 64.257) (width 0.25) (layer "B.Cu") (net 8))
 (segment (start 103.6376 90.3445) (end 109.0191 84.963) (width 0.25) (layer "B.Cu") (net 8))
 (segment (start 128.986 81.28) (end 135.844 81.28) (width 0.25) (layer "B.Cu") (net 8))
 (segment (start 109.0191 84.963) (end 124.1261 84.963) (width 0.25) (layer "B.Cu") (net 8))
 (segment (start 98.0775 90.3445) (end 103.6376 90.3445) (width 0.25) (layer "B.Cu") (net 8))
 (segment (start 128.3976 69.8406) (end 122.814 64.257) (width 0.25) (layer "B.Cu") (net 8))
 (segment (start 135.844 81.28) (end 136.098 81.534) (width 0.25) (layer "B.Cu") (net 8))
 (segment (start 114.518 60.447) (end 115.6449 60.447) (width 0.25) (layer "B.Cu") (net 8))
 (segment (start 128.986 81.28) (end 128.3976 81.28) (width 0.25) (layer "B.Cu") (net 8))
 (segment (start 102.8131 56.388) (end 97.7331 51.308) (width 0.25) (layer "F.Cu") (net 20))
 (segment (start 103.84 56.388) (end 102.8131 56.388) (width 0.25) (layer "F.Cu") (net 20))
 (segment (start 97.7331 51.308) (end 91.394 51.308) (width 0.25) (layer "F.Cu") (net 20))
 (segment (start 115.6622 60.9292) (end 114.8744 61.717) (width 0.25) (layer "F.Cu") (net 4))
 (segment (start 109.682 66.1685) (end 109.682 77.216) (width 0.25) (layer "F.Cu") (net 4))
 (segment (start 114.518 52.827) (end 115.6622 53.9712) (width 0.25) (layer "F.Cu") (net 4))
 (segment (start 114.1335 61.717) (end 109.682 66.1685) (width 0.25) (layer "F.Cu") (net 4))
 (segment (start 114.8744 61.717) (end 114.1335 61.717) (width 0.25) (layer "F.Cu") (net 4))
 (segment (start 115.6622 53.9712) (end 115.6622 60.9292) (width 0.25) (layer "F.Cu") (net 4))
 (segment (start 111.46 48.6421) (end 111.46 44.196) (width 0.25) (layer "B.Cu") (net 4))
 (segment (start 114.518 51.7001) (end 111.46 48.6421) (width 0.25) (layer "B.Cu") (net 4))
 (segment (start 114.518 52.827) (end 114.518 51.7001) (width 0.25) (layer "B.Cu") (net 4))
 (segment (start 134.828 70.104) (end 138.638 70.104) (width 0.25) (layer "B.Cu") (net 18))
 (segment (start 114.508 33.1809) (end 115.6849 34.3578) (width 0.25) (layer "F.Cu") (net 12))
 (segment (start 122.3715 61.5739) (end 122.138 61.5739) (width 0.25) (layer "F.Cu") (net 12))
 (segment (start 122.138 60.447) (end 122.138 59.3201) (width 0.25) (layer "F.Cu") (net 12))
 (segment (start 128.986 86.36) (end 128.986 85.1831) (width 0.25) (layer "F.Cu") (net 12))
 (segment (start 122.138 60.447) (end 122.138 61.5739) (width 0.25) (layer "F.Cu") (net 12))
 (segment (start 124.0075 80.5724) (end 124.0075 63.2099) (width 0.25) (layer "F.Cu") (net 12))
 (segment (start 115.6849 34.3578) (end 115.6849 53.1005) (width 0.25) (layer "F.Cu") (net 12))
 (segment (start 128.986 85.1831) (end 128.6182 85.1831) (width 0.25) (layer "F.Cu") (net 12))
 (segment (start 128.6182 85.1831) (end 124.0075 80.5724) (width 0.25) (layer "F.Cu") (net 12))
 (segment (start 114.508 32.004) (end 114.508 33.1809) (width 0.25) (layer "F.Cu") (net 12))
 (segment (start 124.0075 63.2099) (end 122.3715 61.5739) (width 0.25) (layer "F.Cu") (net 12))
 (segment (start 121.9045 59.3201) (end 122.138 59.3201) (width 0.25) (layer "F.Cu") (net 12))
 (segment (start 115.6849 53.1005) (end 121.9045 59.3201) (width 0.25) (layer "F.Cu") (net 12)))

